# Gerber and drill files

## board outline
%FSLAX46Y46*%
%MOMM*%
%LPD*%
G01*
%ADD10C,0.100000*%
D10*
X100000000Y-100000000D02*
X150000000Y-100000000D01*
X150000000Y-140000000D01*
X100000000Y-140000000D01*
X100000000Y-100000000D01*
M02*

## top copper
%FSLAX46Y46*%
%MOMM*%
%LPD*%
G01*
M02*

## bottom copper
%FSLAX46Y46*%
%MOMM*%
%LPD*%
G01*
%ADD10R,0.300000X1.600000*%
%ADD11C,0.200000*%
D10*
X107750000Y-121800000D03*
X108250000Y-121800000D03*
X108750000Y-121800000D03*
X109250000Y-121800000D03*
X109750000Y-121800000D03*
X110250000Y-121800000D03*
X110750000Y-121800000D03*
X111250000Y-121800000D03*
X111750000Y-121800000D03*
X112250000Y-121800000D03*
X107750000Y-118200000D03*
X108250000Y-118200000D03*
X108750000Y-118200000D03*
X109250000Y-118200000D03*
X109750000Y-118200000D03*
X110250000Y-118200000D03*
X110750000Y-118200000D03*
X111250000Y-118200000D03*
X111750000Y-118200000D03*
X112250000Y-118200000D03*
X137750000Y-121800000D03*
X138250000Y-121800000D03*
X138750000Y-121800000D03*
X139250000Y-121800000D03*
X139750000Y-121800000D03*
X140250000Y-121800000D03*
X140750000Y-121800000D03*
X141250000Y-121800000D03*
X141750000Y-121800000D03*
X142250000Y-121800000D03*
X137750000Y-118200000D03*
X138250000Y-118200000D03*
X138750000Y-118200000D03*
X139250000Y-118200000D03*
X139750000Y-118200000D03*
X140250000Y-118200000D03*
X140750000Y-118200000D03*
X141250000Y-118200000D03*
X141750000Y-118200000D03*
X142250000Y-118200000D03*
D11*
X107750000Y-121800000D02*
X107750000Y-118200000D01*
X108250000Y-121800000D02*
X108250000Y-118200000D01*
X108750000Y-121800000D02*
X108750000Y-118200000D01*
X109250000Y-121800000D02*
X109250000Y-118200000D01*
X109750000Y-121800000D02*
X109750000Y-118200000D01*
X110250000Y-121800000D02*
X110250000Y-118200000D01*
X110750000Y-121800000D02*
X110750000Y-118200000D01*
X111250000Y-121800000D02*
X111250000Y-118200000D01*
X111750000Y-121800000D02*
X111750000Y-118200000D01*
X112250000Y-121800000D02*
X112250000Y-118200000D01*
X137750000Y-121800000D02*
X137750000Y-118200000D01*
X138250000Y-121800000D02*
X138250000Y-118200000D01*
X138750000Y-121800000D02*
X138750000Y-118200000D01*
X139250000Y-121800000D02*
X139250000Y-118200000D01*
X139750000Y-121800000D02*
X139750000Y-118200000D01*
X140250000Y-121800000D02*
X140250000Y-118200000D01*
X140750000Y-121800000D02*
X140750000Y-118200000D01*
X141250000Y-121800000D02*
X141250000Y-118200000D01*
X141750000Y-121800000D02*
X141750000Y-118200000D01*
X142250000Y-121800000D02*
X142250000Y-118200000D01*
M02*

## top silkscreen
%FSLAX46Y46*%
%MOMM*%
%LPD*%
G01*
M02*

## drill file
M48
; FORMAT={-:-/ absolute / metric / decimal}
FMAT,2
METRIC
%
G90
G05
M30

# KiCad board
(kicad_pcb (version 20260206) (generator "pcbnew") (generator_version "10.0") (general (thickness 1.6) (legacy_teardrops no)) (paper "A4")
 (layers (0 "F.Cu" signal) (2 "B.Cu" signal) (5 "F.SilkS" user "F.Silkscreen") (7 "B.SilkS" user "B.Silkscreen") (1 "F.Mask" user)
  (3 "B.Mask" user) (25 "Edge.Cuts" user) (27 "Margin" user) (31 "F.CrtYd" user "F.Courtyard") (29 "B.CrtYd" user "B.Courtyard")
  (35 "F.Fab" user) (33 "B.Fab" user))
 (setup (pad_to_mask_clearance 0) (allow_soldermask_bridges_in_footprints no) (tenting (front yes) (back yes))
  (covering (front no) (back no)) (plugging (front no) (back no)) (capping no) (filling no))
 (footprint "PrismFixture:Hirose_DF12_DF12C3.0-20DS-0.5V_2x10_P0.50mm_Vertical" (layer "B.Cu") (at 110 120)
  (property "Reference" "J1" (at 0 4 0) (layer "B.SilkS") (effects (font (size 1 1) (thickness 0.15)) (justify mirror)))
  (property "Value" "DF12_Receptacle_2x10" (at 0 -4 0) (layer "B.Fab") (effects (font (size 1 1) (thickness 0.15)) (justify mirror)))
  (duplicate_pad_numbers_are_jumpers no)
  (pad "" smd rect (at -2.25 -2) (size 0.28 1.2) (layers "B.Paste"))
  (pad "" smd rect (at -2.25 2) (size 0.28 1.2) (layers "B.Paste"))
  (pad "" smd rect (at -1.75 -2) (size 0.28 1.2) (layers "B.Paste"))
  (pad "" smd rect (at -1.75 2) (size 0.28 1.2) (layers "B.Paste"))
  (pad "" smd rect (at -1.25 -2) (size 0.28 1.2) (layers "B.Paste"))
  (pad "" smd rect (at -1.25 2) (size 0.28 1.2) (layers "B.Paste"))
  (pad "" smd rect (at -0.75 -2) (size 0.28 1.2) (layers "B.Paste"))
  (pad "" smd rect (at -0.75 2) (size 0.28 1.2) (layers "B.Paste"))
  (pad "" smd rect (at -0.25 -2) (size 0.28 1.2) (layers "B.Paste"))
  (pad "" smd rect (at -0.25 2) (size 0.28 1.2) (layers "B.Paste"))
  (pad "" smd rect (at 0.25 -2) (size 0.28 1.2) (layers "B.Paste"))
  (pad "" smd rect (at 0.25 2) (size 0.28 1.2) (layers "B.Paste"))
  (pad "" smd rect (at 0.75 -2) (size 0.28 1.2) (layers "B.Paste"))
  (pad "" smd rect (at 0.75 2) (size 0.28 1.2) (layers "B.Paste"))
  (pad "" smd rect (at 1.25 -2) (size 0.28 1.2) (layers "B.Paste"))
  (pad "" smd rect (at 1.25 2) (size 0.28 1.2) (layers "B.Paste"))
  (pad "" smd rect (at 1.75 -2) (size 0.28 1.2) (layers "B.Paste"))
  (pad "" smd rect (at 1.75 2) (size 0.28 1.2) (layers "B.Paste"))
  (pad "" smd rect (at 2.25 -2) (size 0.28 1.2) (layers "B.Paste"))
  (pad "" smd rect (at 2.25 2) (size 0.28 1.2) (layers "B.Paste"))
  (pad "1" smd rect (at -2.25 1.8) (size 0.3 1.6) (layers "B.Cu" "B.Mask") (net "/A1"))
  (pad "2" smd rect (at -1.75 1.8) (size 0.3 1.6) (layers "B.Cu" "B.Mask") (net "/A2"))
  (pad "3" smd rect (at -1.25 1.8) (size 0.3 1.6) (layers "B.Cu" "B.Mask") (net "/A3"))
  (pad "4" smd rect (at -0.75 1.8) (size 0.3 1.6) (layers "B.Cu" "B.Mask") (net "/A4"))
  (pad "5" smd rect (at -0.25 1.8) (size 0.3 1.6) (layers "B.Cu" "B.Mask") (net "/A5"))
  (pad "6" smd rect (at 0.25 1.8) (size 0.3 1.6) (layers "B.Cu" "B.Mask") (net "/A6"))
  (pad "7" smd rect (at 0.75 1.8) (size 0.3 1.6) (layers "B.Cu" "B.Mask") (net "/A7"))
  (pad "8" smd rect (at 1.25 1.8) (size 0.3 1.6) (layers "B.Cu" "B.Mask") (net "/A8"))
  (pad "9" smd rect (at 1.75 1.8) (size 0.3 1.6) (layers "B.Cu" "B.Mask") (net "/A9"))
  (pad "10" smd rect (at 2.25 1.8) (size 0.3 1.6) (layers "B.Cu" "B.Mask") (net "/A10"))
  (pad "11" smd rect (at -2.25 -1.8) (size 0.3 1.6) (layers "B.Cu" "B.Mask") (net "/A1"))
  (pad "12" smd rect (at -1.75 -1.8) (size 0.3 1.6) (layers "B.Cu" "B.Mask") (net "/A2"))
  (pad "13" smd rect (at -1.25 -1.8) (size 0.3 1.6) (layers "B.Cu" "B.Mask") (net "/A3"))
  (pad "14" smd rect (at -0.75 -1.8) (size 0.3 1.6) (layers "B.Cu" "B.Mask") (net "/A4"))
  (pad "15" smd rect (at -0.25 -1.8) (size 0.3 1.6) (layers "B.Cu" "B.Mask") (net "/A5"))
  (pad "16" smd rect (at 0.25 -1.8) (size 0.3 1.6) (layers "B.Cu" "B.Mask") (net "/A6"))
  (pad "17" smd rect (at 0.75 -1.8) (size 0.3 1.6) (layers "B.Cu" "B.Mask") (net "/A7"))
  (pad "18" smd rect (at 1.25 -1.8) (size 0.3 1.6) (layers "B.Cu" "B.Mask") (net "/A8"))
  (pad "19" smd rect (at 1.75 -1.8) (size 0.3 1.6) (layers "B.Cu" "B.Mask") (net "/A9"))
  (pad "20" smd rect (at 2.25 -1.8) (size 0.3 1.6) (layers "B.Cu" "B.Mask") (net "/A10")))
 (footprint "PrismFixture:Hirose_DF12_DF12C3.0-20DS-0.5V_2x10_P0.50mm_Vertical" (layer "B.Cu") (at 140 120)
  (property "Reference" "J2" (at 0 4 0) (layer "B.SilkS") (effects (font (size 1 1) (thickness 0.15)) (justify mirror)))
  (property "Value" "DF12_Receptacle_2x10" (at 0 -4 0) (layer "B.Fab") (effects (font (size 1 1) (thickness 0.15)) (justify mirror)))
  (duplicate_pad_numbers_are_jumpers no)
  (pad "" smd rect (at -2.25 -2) (size 0.28 1.2) (layers "B.Paste"))
  (pad "" smd rect (at -2.25 2) (size 0.28 1.2) (layers "B.Paste"))
  (pad "" smd rect (at -1.75 -2) (size 0.28 1.2) (layers "B.Paste"))
  (pad "" smd rect (at -1.75 2) (size 0.28 1.2) (layers "B.Paste"))
  (pad "" smd rect (at -1.25 -2) (size 0.28 1.2) (layers "B.Paste"))
  (pad "" smd rect (at -1.25 2) (size 0.28 1.2) (layers "B.Paste"))
  (pad "" smd rect (at -0.75 -2) (size 0.28 1.2) (layers "B.Paste"))
  (pad "" smd rect (at -0.75 2) (size 0.28 1.2) (layers "B.Paste"))
  (pad "" smd rect (at -0.25 -2) (size 0.28 1.2) (layers "B.Paste"))
  (pad "" smd rect (at -0.25 2) (size 0.28 1.2) (layers "B.Paste"))
  (pad "" smd rect (at 0.25 -2) (size 0.28 1.2) (layers "B.Paste"))
  (pad "" smd rect (at 0.25 2) (size 0.28 1.2) (layers "B.Paste"))
  (pad "" smd rect (at 0.75 -2) (size 0.28 1.2) (layers "B.Paste"))
  (pad "" smd rect (at 0.75 2) (size 0.28 1.2) (layers "B.Paste"))
  (pad "" smd rect (at 1.25 -2) (size 0.28 1.2) (layers "B.Paste"))
  (pad "" smd rect (at 1.25 2) (size 0.28 1.2) (layers "B.Paste"))
  (pad "" smd rect (at 1.75 -2) (size 0.28 1.2) (layers "B.Paste"))
  (pad "" smd rect (at 1.75 2) (size 0.28 1.2) (layers "B.Paste"))
  (pad "" smd rect (at 2.25 -2) (size 0.28 1.2) (layers "B.Paste"))
  (pad "" smd rect (at 2.25 2) (size 0.28 1.2) (layers "B.Paste"))
  (pad "1" smd rect (at -2.25 1.8) (size 0.3 1.6) (layers "B.Cu" "B.Mask") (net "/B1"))
  (pad "2" smd rect (at -1.75 1.8) (size 0.3 1.6) (layers "B.Cu" "B.Mask") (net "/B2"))
  (pad "3" smd rect (at -1.25 1.8) (size 0.3 1.6) (layers "B.Cu" "B.Mask") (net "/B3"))
  (pad "4" smd rect (at -0.75 1.8) (size 0.3 1.6) (layers "B.Cu" "B.Mask") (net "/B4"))
  (pad "5" smd rect (at -0.25 1.8) (size 0.3 1.6) (layers "B.Cu" "B.Mask") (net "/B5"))
  (pad "6" smd rect (at 0.25 1.8) (size 0.3 1.6) (layers "B.Cu" "B.Mask") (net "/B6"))
  (pad "7" smd rect (at 0.75 1.8) (size 0.3 1.6) (layers "B.Cu" "B.Mask") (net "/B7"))
  (pad "8" smd rect (at 1.25 1.8) (size 0.3 1.6) (layers "B.Cu" "B.Mask") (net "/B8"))
  (pad "9" smd rect (at 1.75 1.8) (size 0.3 1.6) (layers "B.Cu" "B.Mask") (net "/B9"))
  (pad "10" smd rect (at 2.25 1.8) (size 0.3 1.6) (layers "B.Cu" "B.Mask") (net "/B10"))
  (pad "11" smd rect (at -2.25 -1.8) (size 0.3 1.6) (layers "B.Cu" "B.Mask") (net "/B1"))
  (pad "12" smd rect (at -1.75 -1.8) (size 0.3 1.6) (layers "B.Cu" "B.Mask") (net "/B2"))
  (pad "13" smd rect (at -1.25 -1.8) (size 0.3 1.6) (layers "B.Cu" "B.Mask") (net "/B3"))
  (pad "14" smd rect (at -0.75 -1.8) (size 0.3 1.6) (layers "B.Cu" "B.Mask") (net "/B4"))
  (pad "15" smd rect (at -0.25 -1.8) (size 0.3 1.6) (layers "B.Cu" "B.Mask") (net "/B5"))
  (pad "16" smd rect (at 0.25 -1.8) (size 0.3 1.6) (layers "B.Cu" "B.Mask") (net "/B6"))
  (pad "17" smd rect (at 0.75 -1.8) (size 0.3 1.6) (layers "B.Cu" "B.Mask") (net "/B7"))
  (pad "18" smd rect (at 1.25 -1.8) (size 0.3 1.6) (layers "B.Cu" "B.Mask") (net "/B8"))
  (pad "19" smd rect (at 1.75 -1.8) (size 0.3 1.6) (layers "B.Cu" "B.Mask") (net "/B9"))
  (pad "20" smd rect (at 2.25 -1.8) (size 0.3 1.6) (layers "B.Cu" "B.Mask") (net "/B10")))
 (gr_rect (start 100 100) (end 150 140) (stroke (width 0.1) (type solid)) (fill no) (layer "Edge.Cuts"))
 (segment (start 107.75 121.8) (end 107.75 118.2) (width 0.2) (layer "B.Cu") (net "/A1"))
 (segment (start 108.25 121.8) (end 108.25 118.2) (width 0.2) (layer "B.Cu") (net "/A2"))
 (segment (start 108.75 121.8) (end 108.75 118.2) (width 0.2) (layer "B.Cu") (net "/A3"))
 (segment (start 109.25 121.8) (end 109.25 118.2) (width 0.2) (layer "B.Cu") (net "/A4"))
 (segment (start 109.75 121.8) (end 109.75 118.2) (width 0.2) (layer "B.Cu") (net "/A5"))
 (segment (start 110.25 121.8) (end 110.25 118.2) (width 0.2) (layer "B.Cu") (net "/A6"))
 (segment (start 110.75 121.8) (end 110.75 118.2) (width 0.2) (layer "B.Cu") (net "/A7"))
 (segment (start 111.25 121.8) (end 111.25 118.2) (width 0.2) (layer "B.Cu") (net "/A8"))
 (segment (start 111.75 121.8) (end 111.75 118.2) (width 0.2) (layer "B.Cu") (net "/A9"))
 (segment (start 112.25 121.8) (end 112.25 118.2) (width 0.2) (layer "B.Cu") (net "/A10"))
 (segment (start 137.75 121.8) (end 137.75 118.2) (width 0.2) (layer "B.Cu") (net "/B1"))
 (segment (start 138.25 121.8) (end 138.25 118.2) (width 0.2) (layer "B.Cu") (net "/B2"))
 (segment (start 138.75 121.8) (end 138.75 118.2) (width 0.2) (layer "B.Cu") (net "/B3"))
 (segment (start 139.25 121.8) (end 139.25 118.2) (width 0.2) (layer "B.Cu") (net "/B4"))
 (segment (start 139.75 121.8) (end 139.75 118.2) (width 0.2) (layer "B.Cu") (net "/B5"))
 (segment (start 140.25 121.8) (end 140.25 118.2) (width 0.2) (layer "B.Cu") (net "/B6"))
 (segment (start 140.75 121.8) (end 140.75 118.2) (width 0.2) (layer "B.Cu") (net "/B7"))
 (segment (start 141.25 121.8) (end 141.25 118.2) (width 0.2) (layer "B.Cu") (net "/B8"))
 (segment (start 141.75 121.8) (end 141.75 118.2) (width 0.2) (layer "B.Cu") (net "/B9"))
 (segment (start 142.25 121.8) (end 142.25 118.2) (width 0.2) (layer "B.Cu") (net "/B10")))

